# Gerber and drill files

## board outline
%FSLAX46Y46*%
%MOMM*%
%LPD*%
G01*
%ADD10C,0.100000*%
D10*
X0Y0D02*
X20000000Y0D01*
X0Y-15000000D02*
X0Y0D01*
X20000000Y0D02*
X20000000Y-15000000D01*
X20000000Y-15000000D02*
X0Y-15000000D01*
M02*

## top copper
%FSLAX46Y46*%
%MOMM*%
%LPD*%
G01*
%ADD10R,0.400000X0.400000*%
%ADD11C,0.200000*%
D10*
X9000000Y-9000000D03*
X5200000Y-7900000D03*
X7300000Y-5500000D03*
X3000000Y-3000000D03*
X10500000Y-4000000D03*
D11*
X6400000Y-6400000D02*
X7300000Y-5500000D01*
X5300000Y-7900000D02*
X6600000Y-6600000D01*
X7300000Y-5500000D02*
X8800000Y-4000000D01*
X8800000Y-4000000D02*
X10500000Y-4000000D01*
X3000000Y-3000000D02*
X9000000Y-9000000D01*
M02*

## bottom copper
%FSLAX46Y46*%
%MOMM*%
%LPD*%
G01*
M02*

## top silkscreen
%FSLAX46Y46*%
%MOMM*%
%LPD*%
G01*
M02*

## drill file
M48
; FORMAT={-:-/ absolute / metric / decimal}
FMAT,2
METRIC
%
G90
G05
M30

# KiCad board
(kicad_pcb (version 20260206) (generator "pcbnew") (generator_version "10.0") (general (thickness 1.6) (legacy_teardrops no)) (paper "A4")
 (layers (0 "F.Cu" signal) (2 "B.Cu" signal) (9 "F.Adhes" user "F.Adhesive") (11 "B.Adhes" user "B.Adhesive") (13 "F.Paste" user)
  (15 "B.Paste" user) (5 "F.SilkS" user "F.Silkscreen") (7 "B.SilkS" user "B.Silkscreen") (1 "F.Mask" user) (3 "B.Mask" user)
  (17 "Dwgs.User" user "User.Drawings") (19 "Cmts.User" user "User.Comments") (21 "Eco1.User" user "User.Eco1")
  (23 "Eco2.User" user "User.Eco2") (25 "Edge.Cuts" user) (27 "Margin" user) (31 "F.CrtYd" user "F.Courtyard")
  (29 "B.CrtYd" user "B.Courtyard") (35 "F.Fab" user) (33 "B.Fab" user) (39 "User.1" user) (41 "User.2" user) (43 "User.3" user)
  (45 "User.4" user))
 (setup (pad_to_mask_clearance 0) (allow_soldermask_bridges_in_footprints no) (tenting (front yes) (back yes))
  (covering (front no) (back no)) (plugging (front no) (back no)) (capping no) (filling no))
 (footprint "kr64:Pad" (layer "F.Cu") (at 9 9)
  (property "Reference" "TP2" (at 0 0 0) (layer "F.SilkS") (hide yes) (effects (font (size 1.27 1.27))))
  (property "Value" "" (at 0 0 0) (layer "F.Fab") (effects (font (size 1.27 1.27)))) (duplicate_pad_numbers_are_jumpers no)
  (pad "1" smd rect (at 0 0) (size 0.4 0.4) (layers "F.Cu" "F.Mask" "F.Paste") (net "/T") (thermal_bridge_angle 45)))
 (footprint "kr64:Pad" (layer "F.Cu") (at 5.2 7.9)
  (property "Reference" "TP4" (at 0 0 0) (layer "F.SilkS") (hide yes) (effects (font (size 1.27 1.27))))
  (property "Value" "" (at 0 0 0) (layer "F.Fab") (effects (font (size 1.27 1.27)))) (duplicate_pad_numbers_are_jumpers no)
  (pad "1" smd rect (at 0 0) (size 0.4 0.4) (layers "F.Cu" "F.Mask" "F.Paste") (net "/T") (thermal_bridge_angle 45)))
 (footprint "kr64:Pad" (layer "F.Cu") (at 7.3 5.5)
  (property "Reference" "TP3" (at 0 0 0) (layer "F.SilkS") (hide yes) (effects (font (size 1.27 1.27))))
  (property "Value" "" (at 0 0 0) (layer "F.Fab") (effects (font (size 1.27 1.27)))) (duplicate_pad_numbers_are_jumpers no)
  (pad "1" smd rect (at 0 0) (size 0.4 0.4) (layers "F.Cu" "F.Mask" "F.Paste") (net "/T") (thermal_bridge_angle 45)))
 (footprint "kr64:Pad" (layer "F.Cu") (at 3 3)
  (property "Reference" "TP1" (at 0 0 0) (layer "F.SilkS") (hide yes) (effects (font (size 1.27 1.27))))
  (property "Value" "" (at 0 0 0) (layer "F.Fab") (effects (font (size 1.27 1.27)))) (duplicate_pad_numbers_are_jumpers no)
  (pad "1" smd rect (at 0 0) (size 0.4 0.4) (layers "F.Cu" "F.Mask" "F.Paste") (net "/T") (thermal_bridge_angle 45)))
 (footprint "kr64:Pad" (layer "F.Cu") (at 10.5 4)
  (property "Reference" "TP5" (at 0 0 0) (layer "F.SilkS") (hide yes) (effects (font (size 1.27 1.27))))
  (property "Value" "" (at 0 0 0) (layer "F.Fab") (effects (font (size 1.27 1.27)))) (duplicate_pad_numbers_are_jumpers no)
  (pad "1" smd rect (at 0 0) (size 0.4 0.4) (layers "F.Cu" "F.Mask" "F.Paste") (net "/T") (thermal_bridge_angle 45)))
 (gr_line (start 0 0) (end 20 0) (stroke (width 0.1) (type default)) (layer "Edge.Cuts"))
 (gr_line (start 0 15) (end 0 0) (stroke (width 0.1) (type default)) (layer "Edge.Cuts"))
 (gr_line (start 20 0) (end 20 15) (stroke (width 0.1) (type default)) (layer "Edge.Cuts"))
 (gr_line (start 20 15) (end 0 15) (stroke (width 0.1) (type default)) (layer "Edge.Cuts"))
 (segment (start 6.4 6.4) (end 7.3 5.5) (width 0.2) (layer "F.Cu") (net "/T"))
 (segment (start 5.3 7.9) (end 6.6 6.6) (width 0.2) (layer "F.Cu") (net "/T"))
 (segment (start 7.3 5.5) (end 8.8 4) (width 0.2) (layer "F.Cu") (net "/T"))
 (segment (start 8.8 4) (end 10.5 4) (width 0.2) (layer "F.Cu") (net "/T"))
 (segment (start 3 3) (end 9 9) (width 0.2) (layer "F.Cu") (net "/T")))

